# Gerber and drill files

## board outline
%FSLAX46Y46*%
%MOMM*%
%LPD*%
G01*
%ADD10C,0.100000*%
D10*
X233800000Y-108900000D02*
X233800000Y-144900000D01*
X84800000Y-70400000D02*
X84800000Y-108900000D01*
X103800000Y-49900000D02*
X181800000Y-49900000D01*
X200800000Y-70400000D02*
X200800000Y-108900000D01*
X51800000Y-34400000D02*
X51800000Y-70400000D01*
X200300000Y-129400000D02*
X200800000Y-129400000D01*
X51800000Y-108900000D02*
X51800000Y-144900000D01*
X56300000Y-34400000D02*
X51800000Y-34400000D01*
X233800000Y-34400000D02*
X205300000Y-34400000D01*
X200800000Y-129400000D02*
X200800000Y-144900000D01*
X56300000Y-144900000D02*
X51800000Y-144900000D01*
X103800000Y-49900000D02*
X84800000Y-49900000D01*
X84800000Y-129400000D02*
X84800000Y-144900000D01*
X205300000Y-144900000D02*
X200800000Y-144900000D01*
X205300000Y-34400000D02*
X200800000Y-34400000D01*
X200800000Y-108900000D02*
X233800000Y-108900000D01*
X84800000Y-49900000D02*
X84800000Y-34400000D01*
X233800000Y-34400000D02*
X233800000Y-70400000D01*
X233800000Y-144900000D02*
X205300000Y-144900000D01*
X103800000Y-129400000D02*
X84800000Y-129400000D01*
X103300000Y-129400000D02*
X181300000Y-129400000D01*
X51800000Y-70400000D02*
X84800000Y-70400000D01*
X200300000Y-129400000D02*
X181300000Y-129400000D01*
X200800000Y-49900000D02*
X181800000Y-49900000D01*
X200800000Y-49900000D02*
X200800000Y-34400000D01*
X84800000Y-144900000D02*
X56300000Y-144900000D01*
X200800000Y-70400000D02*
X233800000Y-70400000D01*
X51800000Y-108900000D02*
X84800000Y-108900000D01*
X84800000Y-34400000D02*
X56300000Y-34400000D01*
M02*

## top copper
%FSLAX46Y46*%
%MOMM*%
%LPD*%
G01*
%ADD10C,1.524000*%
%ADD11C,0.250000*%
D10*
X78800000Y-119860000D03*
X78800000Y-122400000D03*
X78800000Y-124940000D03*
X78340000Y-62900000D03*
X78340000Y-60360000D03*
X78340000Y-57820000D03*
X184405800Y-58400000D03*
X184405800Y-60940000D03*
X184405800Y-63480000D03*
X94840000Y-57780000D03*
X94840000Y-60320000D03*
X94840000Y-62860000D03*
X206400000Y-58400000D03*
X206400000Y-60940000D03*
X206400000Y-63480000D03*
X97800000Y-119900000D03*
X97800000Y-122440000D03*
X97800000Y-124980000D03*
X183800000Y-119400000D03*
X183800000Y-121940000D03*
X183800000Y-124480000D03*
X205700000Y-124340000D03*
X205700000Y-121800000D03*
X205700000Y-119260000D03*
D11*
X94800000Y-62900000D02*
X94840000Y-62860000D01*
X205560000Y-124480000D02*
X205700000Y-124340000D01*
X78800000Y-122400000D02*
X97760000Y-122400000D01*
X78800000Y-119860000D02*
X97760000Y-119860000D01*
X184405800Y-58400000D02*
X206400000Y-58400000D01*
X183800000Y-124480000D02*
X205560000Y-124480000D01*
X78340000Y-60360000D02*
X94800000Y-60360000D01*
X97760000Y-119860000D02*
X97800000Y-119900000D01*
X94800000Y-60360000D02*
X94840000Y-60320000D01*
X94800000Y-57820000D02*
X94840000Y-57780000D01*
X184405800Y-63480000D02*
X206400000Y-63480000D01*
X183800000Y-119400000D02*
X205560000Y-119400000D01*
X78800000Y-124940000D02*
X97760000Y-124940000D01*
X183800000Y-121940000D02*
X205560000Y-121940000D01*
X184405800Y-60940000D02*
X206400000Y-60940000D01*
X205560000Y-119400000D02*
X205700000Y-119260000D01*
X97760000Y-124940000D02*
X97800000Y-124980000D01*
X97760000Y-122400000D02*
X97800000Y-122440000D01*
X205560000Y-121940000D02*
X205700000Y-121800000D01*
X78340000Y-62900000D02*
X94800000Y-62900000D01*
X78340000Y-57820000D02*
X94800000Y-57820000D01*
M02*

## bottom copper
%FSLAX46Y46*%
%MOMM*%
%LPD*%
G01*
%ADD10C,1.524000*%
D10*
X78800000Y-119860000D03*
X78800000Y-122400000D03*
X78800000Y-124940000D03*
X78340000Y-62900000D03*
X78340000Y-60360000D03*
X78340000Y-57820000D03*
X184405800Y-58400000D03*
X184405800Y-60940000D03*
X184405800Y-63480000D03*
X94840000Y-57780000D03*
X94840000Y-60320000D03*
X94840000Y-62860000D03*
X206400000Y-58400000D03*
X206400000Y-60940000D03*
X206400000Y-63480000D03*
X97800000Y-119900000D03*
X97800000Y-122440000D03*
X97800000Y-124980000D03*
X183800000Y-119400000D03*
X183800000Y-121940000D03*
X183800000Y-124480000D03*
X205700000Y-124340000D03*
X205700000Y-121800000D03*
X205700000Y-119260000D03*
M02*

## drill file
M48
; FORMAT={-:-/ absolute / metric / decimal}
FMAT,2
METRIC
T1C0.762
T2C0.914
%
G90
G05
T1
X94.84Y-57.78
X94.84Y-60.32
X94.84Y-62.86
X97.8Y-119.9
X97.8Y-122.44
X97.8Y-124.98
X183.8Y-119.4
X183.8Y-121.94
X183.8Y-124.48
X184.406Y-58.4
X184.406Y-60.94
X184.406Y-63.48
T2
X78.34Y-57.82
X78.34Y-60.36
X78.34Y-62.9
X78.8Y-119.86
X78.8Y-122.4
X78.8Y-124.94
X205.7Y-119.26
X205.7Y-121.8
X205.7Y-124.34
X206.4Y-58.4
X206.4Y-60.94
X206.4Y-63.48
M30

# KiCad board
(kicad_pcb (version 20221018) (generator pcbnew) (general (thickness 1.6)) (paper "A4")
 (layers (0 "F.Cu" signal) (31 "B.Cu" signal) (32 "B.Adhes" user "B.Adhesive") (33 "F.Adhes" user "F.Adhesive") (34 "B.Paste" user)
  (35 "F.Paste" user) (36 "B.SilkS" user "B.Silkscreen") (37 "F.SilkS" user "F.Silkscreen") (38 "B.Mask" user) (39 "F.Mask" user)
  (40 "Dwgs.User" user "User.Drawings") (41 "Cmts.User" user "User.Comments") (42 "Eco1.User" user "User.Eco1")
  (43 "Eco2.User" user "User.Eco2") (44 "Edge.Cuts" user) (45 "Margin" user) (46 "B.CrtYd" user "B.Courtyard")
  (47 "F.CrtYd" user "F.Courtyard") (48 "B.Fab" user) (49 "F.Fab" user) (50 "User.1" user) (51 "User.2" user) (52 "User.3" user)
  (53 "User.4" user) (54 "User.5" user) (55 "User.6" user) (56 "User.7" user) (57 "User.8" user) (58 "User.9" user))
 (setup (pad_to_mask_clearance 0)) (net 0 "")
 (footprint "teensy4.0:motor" (layer "F.Cu") (at 77.53 118.59)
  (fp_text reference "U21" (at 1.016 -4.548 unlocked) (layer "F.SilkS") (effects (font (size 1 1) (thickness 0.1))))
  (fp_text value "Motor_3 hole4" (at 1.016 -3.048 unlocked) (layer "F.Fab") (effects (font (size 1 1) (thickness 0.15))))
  (pad "1" thru_hole circle (at 1.27 1.27) (size 1.524 1.524) (drill 0.914) (layers "*.Cu" "*.Mask"))
  (pad "2" thru_hole circle (at 1.27 3.81) (size 1.524 1.524) (drill 0.914) (layers "*.Cu" "*.Mask"))
  (pad "3" thru_hole circle (at 1.27 6.35) (size 1.524 1.524) (drill 0.914) (layers "*.Cu" "*.Mask")))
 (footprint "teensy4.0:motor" (layer "F.Cu") (at 79.61 64.17 180)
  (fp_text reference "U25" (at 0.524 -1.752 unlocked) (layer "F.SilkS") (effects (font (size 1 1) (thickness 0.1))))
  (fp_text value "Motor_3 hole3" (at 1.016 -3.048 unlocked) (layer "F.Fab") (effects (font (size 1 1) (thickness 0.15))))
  (pad "1" thru_hole circle (at 1.27 1.27 180) (size 1.524 1.524) (drill 0.914) (layers "*.Cu" "*.Mask"))
  (pad "2" thru_hole circle (at 1.27 3.81 180) (size 1.524 1.524) (drill 0.914) (layers "*.Cu" "*.Mask"))
  (pad "3" thru_hole circle (at 1.27 6.35 180) (size 1.524 1.524) (drill 0.914) (layers "*.Cu" "*.Mask")))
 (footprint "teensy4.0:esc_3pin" (layer "F.Cu") (at 183.1358 57.13)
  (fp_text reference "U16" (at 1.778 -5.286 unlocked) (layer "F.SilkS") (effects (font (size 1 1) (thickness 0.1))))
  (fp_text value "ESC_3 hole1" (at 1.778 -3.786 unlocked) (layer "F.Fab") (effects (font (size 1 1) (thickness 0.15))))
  (pad "1" thru_hole circle (at 1.27 1.27) (size 1.524 1.524) (drill 0.762) (layers "*.Cu" "*.Mask"))
  (pad "2" thru_hole circle (at 1.27 3.81) (size 1.524 1.524) (drill 0.762) (layers "*.Cu" "*.Mask"))
  (pad "3" thru_hole circle (at 1.27 6.35) (size 1.524 1.524) (drill 0.762) (layers "*.Cu" "*.Mask")))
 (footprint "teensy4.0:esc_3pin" (layer "F.Cu") (at 93.57 56.51)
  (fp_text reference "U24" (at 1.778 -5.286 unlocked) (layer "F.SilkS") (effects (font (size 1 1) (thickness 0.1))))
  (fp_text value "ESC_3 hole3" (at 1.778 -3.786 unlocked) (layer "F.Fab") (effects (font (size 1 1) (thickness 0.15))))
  (pad "1" thru_hole circle (at 1.27 1.27) (size 1.524 1.524) (drill 0.762) (layers "*.Cu" "*.Mask"))
  (pad "2" thru_hole circle (at 1.27 3.81) (size 1.524 1.524) (drill 0.762) (layers "*.Cu" "*.Mask"))
  (pad "3" thru_hole circle (at 1.27 6.35) (size 1.524 1.524) (drill 0.762) (layers "*.Cu" "*.Mask")))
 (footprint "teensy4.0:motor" (layer "F.Cu") (at 205.13 57.13)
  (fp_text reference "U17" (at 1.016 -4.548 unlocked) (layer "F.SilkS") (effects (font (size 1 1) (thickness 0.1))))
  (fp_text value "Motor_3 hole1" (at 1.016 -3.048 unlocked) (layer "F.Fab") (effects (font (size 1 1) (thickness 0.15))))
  (pad "1" thru_hole circle (at 1.27 1.27) (size 1.524 1.524) (drill 0.914) (layers "*.Cu" "*.Mask"))
  (pad "2" thru_hole circle (at 1.27 3.81) (size 1.524 1.524) (drill 0.914) (layers "*.Cu" "*.Mask"))
  (pad "3" thru_hole circle (at 1.27 6.35) (size 1.524 1.524) (drill 0.914) (layers "*.Cu" "*.Mask")))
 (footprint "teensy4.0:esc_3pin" (layer "F.Cu") (at 96.53 118.63)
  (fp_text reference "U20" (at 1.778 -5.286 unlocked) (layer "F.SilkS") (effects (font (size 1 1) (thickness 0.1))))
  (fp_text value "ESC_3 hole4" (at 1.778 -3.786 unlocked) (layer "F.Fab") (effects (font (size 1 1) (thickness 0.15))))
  (pad "1" thru_hole circle (at 1.27 1.27) (size 1.524 1.524) (drill 0.762) (layers "*.Cu" "*.Mask"))
  (pad "2" thru_hole circle (at 1.27 3.81) (size 1.524 1.524) (drill 0.762) (layers "*.Cu" "*.Mask"))
  (pad "3" thru_hole circle (at 1.27 6.35) (size 1.524 1.524) (drill 0.762) (layers "*.Cu" "*.Mask")))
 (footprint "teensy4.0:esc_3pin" (layer "F.Cu") (at 182.53 118.13)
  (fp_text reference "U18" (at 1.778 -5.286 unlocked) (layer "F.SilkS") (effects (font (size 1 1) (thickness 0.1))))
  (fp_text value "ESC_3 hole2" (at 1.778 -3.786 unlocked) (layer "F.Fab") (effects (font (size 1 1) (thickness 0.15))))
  (pad "1" thru_hole circle (at 1.27 1.27) (size 1.524 1.524) (drill 0.762) (layers "*.Cu" "*.Mask"))
  (pad "2" thru_hole circle (at 1.27 3.81) (size 1.524 1.524) (drill 0.762) (layers "*.Cu" "*.Mask"))
  (pad "3" thru_hole circle (at 1.27 6.35) (size 1.524 1.524) (drill 0.762) (layers "*.Cu" "*.Mask")))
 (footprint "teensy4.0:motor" (layer "F.Cu") (at 206.97 125.61 180)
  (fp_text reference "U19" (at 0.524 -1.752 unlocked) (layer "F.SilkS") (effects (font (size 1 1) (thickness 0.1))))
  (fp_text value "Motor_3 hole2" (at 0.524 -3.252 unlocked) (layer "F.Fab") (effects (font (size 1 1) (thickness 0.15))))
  (pad "1" thru_hole circle (at 1.27 1.27 180) (size 1.524 1.524) (drill 0.914) (layers "*.Cu" "*.Mask"))
  (pad "2" thru_hole circle (at 1.27 3.81 180) (size 1.524 1.524) (drill 0.914) (layers "*.Cu" "*.Mask"))
  (pad "3" thru_hole circle (at 1.27 6.35 180) (size 1.524 1.524) (drill 0.914) (layers "*.Cu" "*.Mask")))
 (gr_line (start 233.8 108.9) (end 233.8 144.9) (stroke (width 0.1) (type default)) (layer "Edge.Cuts"))
 (gr_line (start 84.8 70.4) (end 84.8 108.9) (stroke (width 0.1) (type default)) (layer "Edge.Cuts"))
 (gr_line (start 103.8 49.9) (end 181.8 49.9) (stroke (width 0.1) (type default)) (layer "Edge.Cuts"))
 (gr_line (start 200.8 70.4) (end 200.8 108.9) (stroke (width 0.1) (type default)) (layer "Edge.Cuts"))
 (gr_line (start 51.8 34.4) (end 51.8 70.4) (stroke (width 0.1) (type default)) (layer "Edge.Cuts"))
 (gr_line (start 200.3 129.4) (end 200.8 129.4) (stroke (width 0.1) (type default)) (layer "Edge.Cuts"))
 (gr_line (start 51.8 108.9) (end 51.8 144.9) (stroke (width 0.1) (type default)) (layer "Edge.Cuts"))
 (gr_line (start 56.3 34.4) (end 51.8 34.4) (stroke (width 0.1) (type default)) (layer "Edge.Cuts"))
 (gr_line (start 233.8 34.4) (end 205.3 34.4) (stroke (width 0.1) (type default)) (layer "Edge.Cuts"))
 (gr_line (start 200.8 129.4) (end 200.8 144.9) (stroke (width 0.1) (type default)) (layer "Edge.Cuts"))
 (gr_line (start 56.3 144.9) (end 51.8 144.9) (stroke (width 0.1) (type default)) (layer "Edge.Cuts"))
 (gr_line (start 103.8 49.9) (end 84.8 49.9) (stroke (width 0.1) (type default)) (layer "Edge.Cuts"))
 (gr_line (start 84.8 129.4) (end 84.8 144.9) (stroke (width 0.1) (type default)) (layer "Edge.Cuts"))
 (gr_line (start 205.3 144.9) (end 200.8 144.9) (stroke (width 0.1) (type default)) (layer "Edge.Cuts"))
 (gr_line (start 205.3 34.4) (end 200.8 34.4) (stroke (width 0.1) (type default)) (layer "Edge.Cuts"))
 (gr_line (start 200.8 108.9) (end 233.8 108.9) (stroke (width 0.1) (type default)) (layer "Edge.Cuts"))
 (gr_line (start 84.8 49.9) (end 84.8 34.4) (stroke (width 0.1) (type default)) (layer "Edge.Cuts"))
 (gr_line (start 233.8 34.4) (end 233.8 70.4) (stroke (width 0.1) (type default)) (layer "Edge.Cuts"))
 (gr_line (start 233.8 144.9) (end 205.3 144.9) (stroke (width 0.1) (type default)) (layer "Edge.Cuts"))
 (gr_line (start 103.8 129.4) (end 84.8 129.4) (stroke (width 0.1) (type default)) (layer "Edge.Cuts"))
 (gr_line (start 103.3 129.4) (end 181.3 129.4) (stroke (width 0.1) (type default)) (layer "Edge.Cuts"))
 (gr_line (start 51.8 70.4) (end 84.8 70.4) (stroke (width 0.1) (type default)) (layer "Edge.Cuts"))
 (gr_line (start 200.3 129.4) (end 181.3 129.4) (stroke (width 0.1) (type default)) (layer "Edge.Cuts"))
 (gr_line (start 200.8 49.9) (end 181.8 49.9) (stroke (width 0.1) (type default)) (layer "Edge.Cuts"))
 (gr_line (start 200.8 49.9) (end 200.8 34.4) (stroke (width 0.1) (type default)) (layer "Edge.Cuts"))
 (gr_line (start 84.8 144.9) (end 56.3 144.9) (stroke (width 0.1) (type default)) (layer "Edge.Cuts"))
 (gr_line (start 200.8 70.4) (end 233.8 70.4) (stroke (width 0.1) (type default)) (layer "Edge.Cuts"))
 (gr_line (start 51.8 108.9) (end 84.8 108.9) (stroke (width 0.1) (type default)) (layer "Edge.Cuts"))
 (gr_line (start 84.8 34.4) (end 56.3 34.4) (stroke (width 0.1) (type default)) (layer "Edge.Cuts"))
 (segment (start 94.8 62.9) (end 94.84 62.86) (width 0.25) (layer "F.Cu") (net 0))
 (segment (start 205.56 124.48) (end 205.7 124.34) (width 0.25) (layer "F.Cu") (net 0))
 (segment (start 78.8 122.4) (end 97.76 122.4) (width 0.25) (layer "F.Cu") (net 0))
 (segment (start 78.8 119.86) (end 97.76 119.86) (width 0.25) (layer "F.Cu") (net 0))
 (segment (start 184.4058 58.4) (end 206.4 58.4) (width 0.25) (layer "F.Cu") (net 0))
 (segment (start 183.8 124.48) (end 205.56 124.48) (width 0.25) (layer "F.Cu") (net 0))
 (segment (start 78.34 60.36) (end 94.8 60.36) (width 0.25) (layer "F.Cu") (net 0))
 (segment (start 97.76 119.86) (end 97.8 119.9) (width 0.25) (layer "F.Cu") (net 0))
 (segment (start 94.8 60.36) (end 94.84 60.32) (width 0.25) (layer "F.Cu") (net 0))
 (segment (start 94.8 57.82) (end 94.84 57.78) (width 0.25) (layer "F.Cu") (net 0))
 (segment (start 184.4058 63.48) (end 206.4 63.48) (width 0.25) (layer "F.Cu") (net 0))
 (segment (start 183.8 119.4) (end 205.56 119.4) (width 0.25) (layer "F.Cu") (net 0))
 (segment (start 78.8 124.94) (end 97.76 124.94) (width 0.25) (layer "F.Cu") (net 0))
 (segment (start 183.8 121.94) (end 205.56 121.94) (width 0.25) (layer "F.Cu") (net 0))
 (segment (start 184.4058 60.94) (end 206.4 60.94) (width 0.25) (layer "F.Cu") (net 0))
 (segment (start 205.56 119.4) (end 205.7 119.26) (width 0.25) (layer "F.Cu") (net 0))
 (segment (start 97.76 124.94) (end 97.8 124.98) (width 0.25) (layer "F.Cu") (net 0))
 (segment (start 97.76 122.4) (end 97.8 122.44) (width 0.25) (layer "F.Cu") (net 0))
 (segment (start 205.56 121.94) (end 205.7 121.8) (width 0.25) (layer "F.Cu") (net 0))
 (segment (start 78.34 62.9) (end 94.8 62.9) (width 0.25) (layer "F.Cu") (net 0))
 (segment (start 78.34 57.82) (end 94.8 57.82) (width 0.25) (layer "F.Cu") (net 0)))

